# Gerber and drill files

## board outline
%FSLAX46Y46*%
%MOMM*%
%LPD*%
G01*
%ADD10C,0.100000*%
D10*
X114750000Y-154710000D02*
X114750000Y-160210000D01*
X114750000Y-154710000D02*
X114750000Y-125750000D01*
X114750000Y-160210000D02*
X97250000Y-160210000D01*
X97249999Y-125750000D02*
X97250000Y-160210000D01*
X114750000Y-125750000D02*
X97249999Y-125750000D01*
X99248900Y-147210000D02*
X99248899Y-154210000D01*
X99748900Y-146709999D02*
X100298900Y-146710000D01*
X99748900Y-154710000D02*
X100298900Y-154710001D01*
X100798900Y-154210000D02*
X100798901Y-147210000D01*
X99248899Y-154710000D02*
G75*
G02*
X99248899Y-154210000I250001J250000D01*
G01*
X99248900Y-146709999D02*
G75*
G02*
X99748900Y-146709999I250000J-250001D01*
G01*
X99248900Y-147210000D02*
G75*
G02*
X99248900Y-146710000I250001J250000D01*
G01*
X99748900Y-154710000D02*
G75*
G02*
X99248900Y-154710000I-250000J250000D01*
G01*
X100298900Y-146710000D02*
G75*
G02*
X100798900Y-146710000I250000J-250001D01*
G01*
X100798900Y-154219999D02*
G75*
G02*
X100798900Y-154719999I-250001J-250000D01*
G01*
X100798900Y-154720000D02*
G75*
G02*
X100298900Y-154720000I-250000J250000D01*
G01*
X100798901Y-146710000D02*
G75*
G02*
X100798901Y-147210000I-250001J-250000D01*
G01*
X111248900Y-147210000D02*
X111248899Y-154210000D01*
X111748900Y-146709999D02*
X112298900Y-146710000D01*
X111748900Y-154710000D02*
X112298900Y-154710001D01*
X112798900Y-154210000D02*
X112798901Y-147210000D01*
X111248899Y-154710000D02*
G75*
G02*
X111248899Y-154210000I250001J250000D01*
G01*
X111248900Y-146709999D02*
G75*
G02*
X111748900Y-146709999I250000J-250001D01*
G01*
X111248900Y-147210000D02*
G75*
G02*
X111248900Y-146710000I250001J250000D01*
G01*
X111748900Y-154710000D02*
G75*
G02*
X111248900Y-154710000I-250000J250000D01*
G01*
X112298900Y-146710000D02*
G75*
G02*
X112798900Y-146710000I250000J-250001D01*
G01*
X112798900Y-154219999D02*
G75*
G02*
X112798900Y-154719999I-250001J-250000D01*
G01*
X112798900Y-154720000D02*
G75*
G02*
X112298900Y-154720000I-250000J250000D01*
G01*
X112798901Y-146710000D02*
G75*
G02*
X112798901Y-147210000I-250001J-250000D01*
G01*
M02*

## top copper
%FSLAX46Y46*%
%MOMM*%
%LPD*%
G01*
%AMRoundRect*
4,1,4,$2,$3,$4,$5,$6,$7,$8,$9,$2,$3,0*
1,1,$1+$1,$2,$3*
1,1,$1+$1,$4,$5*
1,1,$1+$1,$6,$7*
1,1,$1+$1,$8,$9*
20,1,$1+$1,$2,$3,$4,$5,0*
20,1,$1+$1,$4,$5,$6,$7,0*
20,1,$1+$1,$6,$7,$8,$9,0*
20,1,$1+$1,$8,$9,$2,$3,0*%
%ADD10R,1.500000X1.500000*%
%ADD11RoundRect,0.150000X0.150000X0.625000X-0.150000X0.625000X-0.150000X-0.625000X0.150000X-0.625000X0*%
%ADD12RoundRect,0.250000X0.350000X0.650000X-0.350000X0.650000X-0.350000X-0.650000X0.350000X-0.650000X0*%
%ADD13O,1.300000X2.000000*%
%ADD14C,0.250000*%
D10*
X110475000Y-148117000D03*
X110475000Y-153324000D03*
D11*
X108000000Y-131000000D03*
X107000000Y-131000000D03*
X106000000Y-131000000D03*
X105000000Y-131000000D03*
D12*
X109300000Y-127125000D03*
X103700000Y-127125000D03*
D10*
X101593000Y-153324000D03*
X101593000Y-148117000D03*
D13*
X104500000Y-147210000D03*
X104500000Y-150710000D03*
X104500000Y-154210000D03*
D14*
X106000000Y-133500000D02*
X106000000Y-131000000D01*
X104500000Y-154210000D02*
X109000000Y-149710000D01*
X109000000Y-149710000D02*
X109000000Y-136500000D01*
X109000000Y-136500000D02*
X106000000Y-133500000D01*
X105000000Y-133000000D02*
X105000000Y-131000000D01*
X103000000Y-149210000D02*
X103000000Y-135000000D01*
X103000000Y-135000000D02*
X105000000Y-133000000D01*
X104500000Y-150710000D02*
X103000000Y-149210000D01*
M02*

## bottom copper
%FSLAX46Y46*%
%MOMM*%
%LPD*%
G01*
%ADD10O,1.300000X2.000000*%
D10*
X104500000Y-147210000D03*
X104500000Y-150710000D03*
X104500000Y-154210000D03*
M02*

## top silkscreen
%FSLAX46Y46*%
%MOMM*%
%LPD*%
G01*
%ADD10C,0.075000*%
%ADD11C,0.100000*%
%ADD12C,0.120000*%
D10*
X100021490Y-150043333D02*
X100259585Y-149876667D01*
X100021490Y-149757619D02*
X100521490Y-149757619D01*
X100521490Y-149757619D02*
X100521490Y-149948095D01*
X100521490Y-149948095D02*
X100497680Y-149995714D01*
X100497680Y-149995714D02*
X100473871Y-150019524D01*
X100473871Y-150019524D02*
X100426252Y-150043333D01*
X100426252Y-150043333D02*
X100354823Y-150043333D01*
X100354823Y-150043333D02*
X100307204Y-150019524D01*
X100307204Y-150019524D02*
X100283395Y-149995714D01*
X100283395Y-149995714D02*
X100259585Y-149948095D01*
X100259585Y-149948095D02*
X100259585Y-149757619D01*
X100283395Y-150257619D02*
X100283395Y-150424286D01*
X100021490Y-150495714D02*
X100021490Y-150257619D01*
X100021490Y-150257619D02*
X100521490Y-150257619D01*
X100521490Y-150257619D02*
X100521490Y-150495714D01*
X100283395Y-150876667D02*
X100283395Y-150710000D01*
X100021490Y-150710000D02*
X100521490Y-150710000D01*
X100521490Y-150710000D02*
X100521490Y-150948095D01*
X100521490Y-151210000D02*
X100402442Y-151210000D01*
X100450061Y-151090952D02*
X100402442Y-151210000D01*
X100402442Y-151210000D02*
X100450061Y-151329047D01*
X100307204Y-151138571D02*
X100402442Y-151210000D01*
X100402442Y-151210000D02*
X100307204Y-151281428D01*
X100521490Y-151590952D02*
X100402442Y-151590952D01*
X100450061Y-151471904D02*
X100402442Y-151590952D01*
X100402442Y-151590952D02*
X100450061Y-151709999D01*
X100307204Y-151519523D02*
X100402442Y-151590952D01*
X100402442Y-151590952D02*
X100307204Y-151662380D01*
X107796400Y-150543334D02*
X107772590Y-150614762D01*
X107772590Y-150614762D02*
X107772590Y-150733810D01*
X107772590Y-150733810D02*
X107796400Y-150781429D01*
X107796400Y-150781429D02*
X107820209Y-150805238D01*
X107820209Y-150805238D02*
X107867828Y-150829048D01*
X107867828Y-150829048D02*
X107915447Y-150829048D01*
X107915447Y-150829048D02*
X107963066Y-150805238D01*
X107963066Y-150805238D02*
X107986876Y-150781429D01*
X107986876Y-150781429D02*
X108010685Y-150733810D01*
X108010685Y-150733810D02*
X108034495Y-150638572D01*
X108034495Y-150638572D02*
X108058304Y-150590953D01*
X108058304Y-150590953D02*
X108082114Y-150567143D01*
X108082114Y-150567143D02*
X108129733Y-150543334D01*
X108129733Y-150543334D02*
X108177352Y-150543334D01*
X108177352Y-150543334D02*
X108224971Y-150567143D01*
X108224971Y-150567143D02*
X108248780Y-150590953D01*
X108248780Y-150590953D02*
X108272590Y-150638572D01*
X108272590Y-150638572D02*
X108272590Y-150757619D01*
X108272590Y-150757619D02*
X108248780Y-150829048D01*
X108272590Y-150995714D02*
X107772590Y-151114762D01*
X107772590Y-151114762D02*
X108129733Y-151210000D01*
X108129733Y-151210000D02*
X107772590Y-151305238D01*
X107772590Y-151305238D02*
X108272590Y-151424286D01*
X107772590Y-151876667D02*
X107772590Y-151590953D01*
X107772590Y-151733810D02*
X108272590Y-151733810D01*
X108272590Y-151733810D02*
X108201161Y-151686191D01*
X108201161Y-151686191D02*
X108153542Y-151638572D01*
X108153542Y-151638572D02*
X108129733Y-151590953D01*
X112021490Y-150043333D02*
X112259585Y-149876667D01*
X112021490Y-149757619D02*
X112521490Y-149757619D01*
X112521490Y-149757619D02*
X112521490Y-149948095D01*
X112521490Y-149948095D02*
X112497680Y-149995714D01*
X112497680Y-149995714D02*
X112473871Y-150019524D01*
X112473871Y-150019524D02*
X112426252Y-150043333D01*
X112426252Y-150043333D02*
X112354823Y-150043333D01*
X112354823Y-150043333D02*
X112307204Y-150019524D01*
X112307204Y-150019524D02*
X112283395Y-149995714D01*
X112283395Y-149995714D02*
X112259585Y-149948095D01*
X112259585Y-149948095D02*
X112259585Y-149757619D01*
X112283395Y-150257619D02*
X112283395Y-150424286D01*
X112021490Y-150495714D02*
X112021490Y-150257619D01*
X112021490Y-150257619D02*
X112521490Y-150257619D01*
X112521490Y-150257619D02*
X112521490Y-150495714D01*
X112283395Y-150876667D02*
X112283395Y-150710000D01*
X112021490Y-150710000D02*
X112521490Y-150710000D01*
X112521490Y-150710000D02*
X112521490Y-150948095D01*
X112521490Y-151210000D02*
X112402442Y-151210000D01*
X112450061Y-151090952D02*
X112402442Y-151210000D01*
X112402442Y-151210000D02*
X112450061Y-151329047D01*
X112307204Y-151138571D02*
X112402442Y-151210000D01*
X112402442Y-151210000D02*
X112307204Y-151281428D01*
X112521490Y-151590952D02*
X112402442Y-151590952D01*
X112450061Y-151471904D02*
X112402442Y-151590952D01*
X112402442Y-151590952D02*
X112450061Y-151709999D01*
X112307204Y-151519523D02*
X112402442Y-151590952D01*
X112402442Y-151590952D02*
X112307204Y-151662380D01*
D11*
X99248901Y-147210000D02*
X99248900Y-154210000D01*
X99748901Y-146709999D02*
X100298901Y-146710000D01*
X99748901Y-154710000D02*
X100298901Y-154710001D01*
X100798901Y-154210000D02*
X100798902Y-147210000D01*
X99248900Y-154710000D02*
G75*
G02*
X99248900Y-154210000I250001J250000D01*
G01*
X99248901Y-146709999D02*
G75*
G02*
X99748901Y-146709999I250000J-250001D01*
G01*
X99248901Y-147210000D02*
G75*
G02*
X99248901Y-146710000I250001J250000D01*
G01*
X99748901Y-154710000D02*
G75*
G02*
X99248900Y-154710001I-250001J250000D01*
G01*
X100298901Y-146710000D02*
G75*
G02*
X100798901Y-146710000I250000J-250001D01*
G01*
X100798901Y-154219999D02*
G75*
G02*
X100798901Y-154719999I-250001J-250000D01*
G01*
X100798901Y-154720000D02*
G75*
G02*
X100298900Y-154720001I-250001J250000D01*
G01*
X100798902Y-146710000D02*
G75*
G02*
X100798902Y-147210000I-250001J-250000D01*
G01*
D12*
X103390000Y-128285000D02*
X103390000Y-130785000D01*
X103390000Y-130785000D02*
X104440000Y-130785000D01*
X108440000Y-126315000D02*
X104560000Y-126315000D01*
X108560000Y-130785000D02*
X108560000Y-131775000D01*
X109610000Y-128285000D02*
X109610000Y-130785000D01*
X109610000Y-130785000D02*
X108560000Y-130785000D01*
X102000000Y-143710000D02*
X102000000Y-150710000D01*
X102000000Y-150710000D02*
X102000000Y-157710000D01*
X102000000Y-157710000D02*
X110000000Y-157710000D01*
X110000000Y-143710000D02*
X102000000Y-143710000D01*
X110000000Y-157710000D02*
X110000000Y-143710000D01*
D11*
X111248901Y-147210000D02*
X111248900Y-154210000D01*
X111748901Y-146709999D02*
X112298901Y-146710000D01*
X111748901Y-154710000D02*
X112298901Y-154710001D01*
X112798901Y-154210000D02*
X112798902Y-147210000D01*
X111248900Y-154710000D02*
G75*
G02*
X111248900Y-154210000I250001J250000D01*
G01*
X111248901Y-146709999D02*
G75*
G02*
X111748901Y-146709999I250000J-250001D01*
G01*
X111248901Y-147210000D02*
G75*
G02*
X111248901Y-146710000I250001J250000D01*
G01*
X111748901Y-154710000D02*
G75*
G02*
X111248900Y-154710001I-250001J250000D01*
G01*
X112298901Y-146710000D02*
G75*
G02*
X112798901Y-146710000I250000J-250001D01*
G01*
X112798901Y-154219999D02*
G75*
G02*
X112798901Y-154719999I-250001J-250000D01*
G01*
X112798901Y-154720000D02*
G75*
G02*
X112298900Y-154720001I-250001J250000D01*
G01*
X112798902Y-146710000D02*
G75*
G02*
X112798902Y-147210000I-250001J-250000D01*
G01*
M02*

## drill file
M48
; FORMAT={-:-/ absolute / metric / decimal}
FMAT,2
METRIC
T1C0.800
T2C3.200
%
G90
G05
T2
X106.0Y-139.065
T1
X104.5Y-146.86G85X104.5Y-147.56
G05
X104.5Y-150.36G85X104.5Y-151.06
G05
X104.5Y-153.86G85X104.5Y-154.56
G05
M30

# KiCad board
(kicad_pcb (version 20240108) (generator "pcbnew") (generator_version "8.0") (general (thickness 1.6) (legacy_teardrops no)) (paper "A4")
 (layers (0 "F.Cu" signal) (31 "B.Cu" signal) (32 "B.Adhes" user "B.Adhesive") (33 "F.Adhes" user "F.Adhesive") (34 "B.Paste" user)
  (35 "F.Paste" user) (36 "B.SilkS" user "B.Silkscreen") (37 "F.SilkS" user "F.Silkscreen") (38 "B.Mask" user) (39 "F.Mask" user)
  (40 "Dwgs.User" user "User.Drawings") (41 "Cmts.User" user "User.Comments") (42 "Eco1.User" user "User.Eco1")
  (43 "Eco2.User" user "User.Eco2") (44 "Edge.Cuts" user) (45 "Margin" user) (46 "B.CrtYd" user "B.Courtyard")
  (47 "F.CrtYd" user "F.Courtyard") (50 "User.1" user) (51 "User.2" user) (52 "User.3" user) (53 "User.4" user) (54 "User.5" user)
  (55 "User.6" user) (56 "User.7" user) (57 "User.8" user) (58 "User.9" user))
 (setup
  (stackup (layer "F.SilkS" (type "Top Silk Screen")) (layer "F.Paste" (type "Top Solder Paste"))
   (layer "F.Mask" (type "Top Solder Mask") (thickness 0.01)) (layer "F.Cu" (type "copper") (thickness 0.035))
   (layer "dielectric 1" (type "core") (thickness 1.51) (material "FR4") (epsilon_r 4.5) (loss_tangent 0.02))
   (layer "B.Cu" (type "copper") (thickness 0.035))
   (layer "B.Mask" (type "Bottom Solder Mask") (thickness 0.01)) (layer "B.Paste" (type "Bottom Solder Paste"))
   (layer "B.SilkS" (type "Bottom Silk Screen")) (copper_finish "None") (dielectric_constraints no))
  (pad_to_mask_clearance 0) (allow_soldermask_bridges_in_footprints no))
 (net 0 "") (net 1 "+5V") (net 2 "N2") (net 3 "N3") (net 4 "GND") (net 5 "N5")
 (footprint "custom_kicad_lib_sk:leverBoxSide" (layer "F.Cu") (at 100 150.71 -90)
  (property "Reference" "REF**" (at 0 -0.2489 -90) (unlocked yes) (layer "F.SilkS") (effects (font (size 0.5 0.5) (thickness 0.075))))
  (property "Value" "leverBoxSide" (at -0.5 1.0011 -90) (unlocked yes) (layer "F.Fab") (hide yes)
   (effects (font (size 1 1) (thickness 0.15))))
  (fp_line (start -3.5 0.751099) (end 3.5 0.7511) (stroke (width 0.1) (type default)) (layer "F.SilkS"))
  (fp_line (start -4.000001 0.251099) (end -4 -0.298901) (stroke (width 0.1) (type default)) (layer "F.SilkS"))
  (fp_line (start 4 0.251099) (end 4.000001 -0.298901) (stroke (width 0.1) (type default)) (layer "F.SilkS"))
  (fp_line (start 3.5 -0.798901) (end -3.5 -0.798902) (stroke (width 0.1) (type default)) (layer "F.SilkS"))
  (fp_arc (start 4 0.7511) (mid 3.75 0.854653) (end 3.5 0.7511) (stroke (width 0.1) (type default)) (layer "F.SilkS"))
  (fp_arc (start -4.000001 0.751099) (mid -4.103554 0.501099) (end -4.000001 0.251099) (stroke (width 0.1) (type default)) (layer "F.SilkS"))
  (fp_arc (start -3.5 0.751099) (mid -3.75 0.854652) (end -4 0.751099) (stroke (width 0.1) (type default)) (layer "F.SilkS"))
  (fp_arc (start 4 0.251099) (mid 4.103554 0.501099) (end 4 0.751099) (stroke (width 0.1) (type default)) (layer "F.SilkS"))
  (fp_arc (start -4 -0.298901) (mid -4.103553 -0.548901) (end -4 -0.798901) (stroke (width 0.1) (type default)) (layer "F.SilkS"))
  (fp_arc (start 3.509999 -0.798901) (mid 3.759999 -0.902454) (end 4.009999 -0.798901) (stroke (width 0.1) (type default)) (layer "F.SilkS"))
  (fp_arc (start 4.01 -0.798901) (mid 4.113554 -0.548901) (end 4.01 -0.298901) (stroke (width 0.1) (type default)) (layer "F.SilkS"))
  (fp_arc (start -4 -0.798902) (mid -3.75 -0.902455) (end -3.5 -0.798902) (stroke (width 0.1) (type default)) (layer "F.SilkS"))
  (fp_line (start -3.5 0.7511) (end 3.5 0.751101) (stroke (width 0.1) (type default)) (layer "Edge.Cuts"))
  (fp_line (start -4.000001 0.2511) (end -4 -0.2989) (stroke (width 0.1) (type default)) (layer "Edge.Cuts"))
  (fp_line (start 4 0.2511) (end 4.000001 -0.2989) (stroke (width 0.1) (type default)) (layer "Edge.Cuts"))
  (fp_line (start 3.5 -0.7989) (end -3.5 -0.798901) (stroke (width 0.1) (type default)) (layer "Edge.Cuts"))
  (fp_arc (start 4 0.751101) (mid 3.75 0.854654) (end 3.5 0.751101) (stroke (width 0.1) (type default)) (layer "Edge.Cuts"))
  (fp_arc (start -4.000001 0.7511) (mid -4.103554 0.5011) (end -4.000001 0.2511) (stroke (width 0.1) (type default)) (layer "Edge.Cuts"))
  (fp_arc (start -3.5 0.7511) (mid -3.75 0.854653) (end -4 0.7511) (stroke (width 0.1) (type default)) (layer "Edge.Cuts"))
  (fp_arc (start 4 0.2511) (mid 4.103553 0.5011) (end 4 0.7511) (stroke (width 0.1) (type default)) (layer "Edge.Cuts"))
  (fp_arc (start -4 -0.2989) (mid -4.103553 -0.5489) (end -4 -0.7989) (stroke (width 0.1) (type default)) (layer "Edge.Cuts"))
  (fp_arc (start 3.509999 -0.7989) (mid 3.759999 -0.902453) (end 4.009999 -0.7989) (stroke (width 0.1) (type default)) (layer "Edge.Cuts"))
  (fp_arc (start 4.01 -0.7989) (mid 4.113553 -0.5489) (end 4.01 -0.2989) (stroke (width 0.1) (type default)) (layer "Edge.Cuts"))
  (fp_arc (start -4 -0.798901) (mid -3.75 -0.902454) (end -3.5 -0.798901) (stroke (width 0.1) (type default)) (layer "Edge.Cuts")))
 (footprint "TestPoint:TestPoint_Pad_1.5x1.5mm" (layer "F.Cu") (at 110.475 148.117 180)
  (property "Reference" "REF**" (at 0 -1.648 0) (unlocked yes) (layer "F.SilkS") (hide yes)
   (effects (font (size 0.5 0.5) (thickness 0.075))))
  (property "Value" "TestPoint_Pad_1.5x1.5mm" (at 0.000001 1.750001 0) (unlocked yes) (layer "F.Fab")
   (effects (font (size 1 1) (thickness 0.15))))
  (pad "1" smd rect (at 0 0 180) (size 1.5 1.5) (layers "F.Cu" "F.Mask")))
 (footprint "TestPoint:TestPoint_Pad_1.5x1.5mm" (layer "F.Cu") (at 110.475 153.324 180)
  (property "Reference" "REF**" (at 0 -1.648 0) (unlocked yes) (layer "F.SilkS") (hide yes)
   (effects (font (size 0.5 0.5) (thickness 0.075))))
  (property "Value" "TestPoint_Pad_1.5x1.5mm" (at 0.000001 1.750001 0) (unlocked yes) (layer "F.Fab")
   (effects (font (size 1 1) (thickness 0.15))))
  (pad "1" smd rect (at 0 0 180) (size 1.5 1.5) (layers "F.Cu" "F.Mask")))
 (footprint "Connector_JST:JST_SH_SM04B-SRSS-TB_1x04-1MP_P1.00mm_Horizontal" (layer "F.Cu") (at 106.5 129 180)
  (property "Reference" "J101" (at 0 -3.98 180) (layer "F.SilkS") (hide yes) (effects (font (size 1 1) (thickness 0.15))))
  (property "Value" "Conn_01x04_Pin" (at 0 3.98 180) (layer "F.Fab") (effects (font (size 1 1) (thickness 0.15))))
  (fp_line (start 3.11 0.715) (end 3.11 -1.785) (stroke (width 0.12) (type solid)) (layer "F.SilkS"))
  (fp_line (start 3.11 -1.785) (end 2.06 -1.785) (stroke (width 0.12) (type solid)) (layer "F.SilkS"))
  (fp_line (start -1.94 2.685) (end 1.94 2.685) (stroke (width 0.12) (type solid)) (layer "F.SilkS"))
  (fp_line (start -2.06 -1.785) (end -2.06 -2.775) (stroke (width 0.12) (type solid)) (layer "F.SilkS"))
  (fp_line (start -3.11 0.715) (end -3.11 -1.785) (stroke (width 0.12) (type solid)) (layer "F.SilkS"))
  (fp_line (start -3.11 -1.785) (end -2.06 -1.785) (stroke (width 0.12) (type solid)) (layer "F.SilkS"))
  (pad "1" smd roundrect (at -1.5 -2 180) (size 0.6 1.55) (layers "F.Cu" "F.Paste" "F.Mask") (roundrect_rratio 0.25) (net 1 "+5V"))
  (pad "2" smd roundrect (at -0.5 -2 180) (size 0.6 1.55) (layers "F.Cu" "F.Paste" "F.Mask") (roundrect_rratio 0.25) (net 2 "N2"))
  (pad "3" smd roundrect (at 0.5 -2 180) (size 0.6 1.55) (layers "F.Cu" "F.Paste" "F.Mask") (roundrect_rratio 0.25) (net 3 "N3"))
  (pad "4" smd roundrect (at 1.5 -2 180) (size 0.6 1.55) (layers "F.Cu" "F.Paste" "F.Mask") (roundrect_rratio 0.25) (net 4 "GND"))
  (pad "MP" smd roundrect (at -2.8 1.875 180) (size 1.2 1.8) (layers "F.Cu" "F.Paste" "F.Mask") (roundrect_rratio 0.208333))
  (pad "MP" smd roundrect (at 2.8 1.875 180) (size 1.2 1.8) (layers "F.Cu" "F.Paste" "F.Mask") (roundrect_rratio 0.208333)))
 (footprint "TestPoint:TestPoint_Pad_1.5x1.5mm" (layer "F.Cu") (at 101.593 153.324 180)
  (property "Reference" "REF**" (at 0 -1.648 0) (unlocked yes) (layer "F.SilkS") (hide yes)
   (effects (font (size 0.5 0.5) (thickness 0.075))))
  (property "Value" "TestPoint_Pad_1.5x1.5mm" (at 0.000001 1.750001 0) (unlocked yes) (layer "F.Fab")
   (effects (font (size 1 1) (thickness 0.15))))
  (pad "1" smd rect (at 0 0 180) (size 1.5 1.5) (layers "F.Cu" "F.Mask")))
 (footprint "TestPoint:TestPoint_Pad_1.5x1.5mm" (layer "F.Cu") (at 101.593 148.117 180)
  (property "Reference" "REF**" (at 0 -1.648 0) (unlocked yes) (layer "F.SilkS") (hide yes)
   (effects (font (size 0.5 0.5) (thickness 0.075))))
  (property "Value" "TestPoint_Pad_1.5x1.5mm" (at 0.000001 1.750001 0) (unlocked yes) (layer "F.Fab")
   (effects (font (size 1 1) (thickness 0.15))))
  (pad "1" smd rect (at 0 0 180) (size 1.5 1.5) (layers "F.Cu" "F.Mask")))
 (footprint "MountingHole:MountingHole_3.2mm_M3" (layer "F.Cu") (at 106 139.065)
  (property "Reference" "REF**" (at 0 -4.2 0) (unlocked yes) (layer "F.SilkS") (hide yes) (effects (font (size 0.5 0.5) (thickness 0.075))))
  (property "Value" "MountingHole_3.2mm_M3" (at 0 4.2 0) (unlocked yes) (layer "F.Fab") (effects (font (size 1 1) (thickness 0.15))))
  (pad "" np_thru_hole circle (at 0 0) (size 3.2 3.2) (drill 3.2) (layers "*.Cu" "*.Mask")))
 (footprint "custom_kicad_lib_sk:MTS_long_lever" (layer "F.Cu") (at 107.5 151.21 -90)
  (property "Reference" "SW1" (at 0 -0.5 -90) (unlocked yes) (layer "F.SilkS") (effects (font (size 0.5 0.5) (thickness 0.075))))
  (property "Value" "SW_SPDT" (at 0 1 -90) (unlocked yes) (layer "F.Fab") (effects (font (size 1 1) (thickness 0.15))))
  (fp_line (start -7.5 5.5) (end -0.5 5.5) (stroke (width 0.12) (type solid)) (layer "F.SilkS"))
  (fp_line (start -0.5 5.5) (end 6.5 5.5) (stroke (width 0.12) (type solid)) (layer "F.SilkS"))
  (fp_line (start 6.5 5.5) (end 6.5 -2.5) (stroke (width 0.12) (type solid)) (layer "F.SilkS"))
  (fp_line (start -7.5 -2.5) (end -7.5 5.5) (stroke (width 0.12) (type solid)) (layer "F.SilkS"))
  (fp_line (start 6.5 -2.5) (end -7.5 -2.5) (stroke (width 0.12) (type solid)) (layer "F.SilkS"))
  (pad "1" thru_hole oval (at -4 3 270) (size 2 1.3) (drill oval 1.5 0.8) (layers "*.Cu" "*.Mask") (remove_unused_layers no) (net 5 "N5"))
  (pad "2" thru_hole oval (at -0.5 3 270) (size 2 1.3) (drill oval 1.5 0.8) (layers "*.Cu" "*.Mask") (remove_unused_layers no) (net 4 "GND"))
  (pad "3" thru_hole oval (at 3 3 270) (size 2 1.3) (drill oval 1.5 0.8) (layers "*.Cu" "*.Mask") (remove_unused_layers no) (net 3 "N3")))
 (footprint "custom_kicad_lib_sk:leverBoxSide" (layer "F.Cu") (at 112 150.71 -90)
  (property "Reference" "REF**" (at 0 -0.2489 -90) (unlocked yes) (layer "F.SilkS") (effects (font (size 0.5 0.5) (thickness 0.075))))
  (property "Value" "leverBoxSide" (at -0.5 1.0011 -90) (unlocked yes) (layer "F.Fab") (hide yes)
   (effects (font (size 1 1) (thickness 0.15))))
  (fp_line (start -3.5 0.751099) (end 3.5 0.7511) (stroke (width 0.1) (type default)) (layer "F.SilkS"))
  (fp_line (start -4.000001 0.251099) (end -4 -0.298901) (stroke (width 0.1) (type default)) (layer "F.SilkS"))
  (fp_line (start 4 0.251099) (end 4.000001 -0.298901) (stroke (width 0.1) (type default)) (layer "F.SilkS"))
  (fp_line (start 3.5 -0.798901) (end -3.5 -0.798902) (stroke (width 0.1) (type default)) (layer "F.SilkS"))
  (fp_arc (start 4 0.7511) (mid 3.75 0.854653) (end 3.5 0.7511) (stroke (width 0.1) (type default)) (layer "F.SilkS"))
  (fp_arc (start -4.000001 0.751099) (mid -4.103554 0.501099) (end -4.000001 0.251099) (stroke (width 0.1) (type default)) (layer "F.SilkS"))
  (fp_arc (start -3.5 0.751099) (mid -3.75 0.854652) (end -4 0.751099) (stroke (width 0.1) (type default)) (layer "F.SilkS"))
  (fp_arc (start 4 0.251099) (mid 4.103554 0.501099) (end 4 0.751099) (stroke (width 0.1) (type default)) (layer "F.SilkS"))
  (fp_arc (start -4 -0.298901) (mid -4.103553 -0.548901) (end -4 -0.798901) (stroke (width 0.1) (type default)) (layer "F.SilkS"))
  (fp_arc (start 3.509999 -0.798901) (mid 3.759999 -0.902454) (end 4.009999 -0.798901) (stroke (width 0.1) (type default)) (layer "F.SilkS"))
  (fp_arc (start 4.01 -0.798901) (mid 4.113554 -0.548901) (end 4.01 -0.298901) (stroke (width 0.1) (type default)) (layer "F.SilkS"))
  (fp_arc (start -4 -0.798902) (mid -3.75 -0.902455) (end -3.5 -0.798902) (stroke (width 0.1) (type default)) (layer "F.SilkS"))
  (fp_line (start -3.5 0.7511) (end 3.5 0.751101) (stroke (width 0.1) (type default)) (layer "Edge.Cuts"))
  (fp_line (start -4.000001 0.2511) (end -4 -0.2989) (stroke (width 0.1) (type default)) (layer "Edge.Cuts"))
  (fp_line (start 4 0.2511) (end 4.000001 -0.2989) (stroke (width 0.1) (type default)) (layer "Edge.Cuts"))
  (fp_line (start 3.5 -0.7989) (end -3.5 -0.798901) (stroke (width 0.1) (type default)) (layer "Edge.Cuts"))
  (fp_arc (start 4 0.751101) (mid 3.75 0.854654) (end 3.5 0.751101) (stroke (width 0.1) (type default)) (layer "Edge.Cuts"))
  (fp_arc (start -4.000001 0.7511) (mid -4.103554 0.5011) (end -4.000001 0.2511) (stroke (width 0.1) (type default)) (layer "Edge.Cuts"))
  (fp_arc (start -3.5 0.7511) (mid -3.75 0.854653) (end -4 0.7511) (stroke (width 0.1) (type default)) (layer "Edge.Cuts"))
  (fp_arc (start 4 0.2511) (mid 4.103553 0.5011) (end 4 0.7511) (stroke (width 0.1) (type default)) (layer "Edge.Cuts"))
  (fp_arc (start -4 -0.2989) (mid -4.103553 -0.5489) (end -4 -0.7989) (stroke (width 0.1) (type default)) (layer "Edge.Cuts"))
  (fp_arc (start 3.509999 -0.7989) (mid 3.759999 -0.902453) (end 4.009999 -0.7989) (stroke (width 0.1) (type default)) (layer "Edge.Cuts"))
  (fp_arc (start 4.01 -0.7989) (mid 4.113553 -0.5489) (end 4.01 -0.2989) (stroke (width 0.1) (type default)) (layer "Edge.Cuts"))
  (fp_arc (start -4 -0.798901) (mid -3.75 -0.902454) (end -3.5 -0.798901) (stroke (width 0.1) (type default)) (layer "Edge.Cuts")))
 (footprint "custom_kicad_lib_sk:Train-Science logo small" (layer "B.Cu") (at 106 131.5 180)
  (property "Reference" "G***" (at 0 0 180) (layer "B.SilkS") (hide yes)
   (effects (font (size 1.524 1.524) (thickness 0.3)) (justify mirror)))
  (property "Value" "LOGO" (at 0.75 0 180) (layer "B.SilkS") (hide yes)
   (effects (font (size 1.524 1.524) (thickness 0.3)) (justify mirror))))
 (gr_line (start 114.75 154.71) (end 114.75 160.21) (stroke (width 0.1) (type default)) (layer "Edge.Cuts"))
 (gr_line (start 114.75 154.71) (end 114.75 125.75) (stroke (width 0.1) (type default)) (layer "Edge.Cuts"))
 (gr_line (start 114.75 160.21) (end 97.25 160.21) (stroke (width 0.1) (type default)) (layer "Edge.Cuts"))
 (gr_line (start 97.249999 125.75) (end 97.25 160.21) (stroke (width 0.1) (type default)) (layer "Edge.Cuts"))
 (gr_line (start 114.75 125.75) (end 97.249999 125.75) (stroke (width 0.1) (type default)) (layer "Edge.Cuts"))
 (segment (start 106 133.5) (end 106 131) (width 0.25) (layer "F.Cu") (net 3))
 (segment (start 104.5 154.21) (end 109 149.71) (width 0.25) (layer "F.Cu") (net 3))
 (segment (start 109 149.71) (end 109 136.5) (width 0.25) (layer "F.Cu") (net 3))
 (segment (start 109 136.5) (end 106 133.5) (width 0.25) (layer "F.Cu") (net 3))
 (segment (start 105 133) (end 105 131) (width 0.25) (layer "F.Cu") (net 4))
 (segment (start 103 149.21) (end 103 135) (width 0.25) (layer "F.Cu") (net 4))
 (segment (start 103 135) (end 105 133) (width 0.25) (layer "F.Cu") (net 4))
 (segment (start 104.5 150.71) (end 103 149.21) (width 0.25) (layer "F.Cu") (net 4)))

